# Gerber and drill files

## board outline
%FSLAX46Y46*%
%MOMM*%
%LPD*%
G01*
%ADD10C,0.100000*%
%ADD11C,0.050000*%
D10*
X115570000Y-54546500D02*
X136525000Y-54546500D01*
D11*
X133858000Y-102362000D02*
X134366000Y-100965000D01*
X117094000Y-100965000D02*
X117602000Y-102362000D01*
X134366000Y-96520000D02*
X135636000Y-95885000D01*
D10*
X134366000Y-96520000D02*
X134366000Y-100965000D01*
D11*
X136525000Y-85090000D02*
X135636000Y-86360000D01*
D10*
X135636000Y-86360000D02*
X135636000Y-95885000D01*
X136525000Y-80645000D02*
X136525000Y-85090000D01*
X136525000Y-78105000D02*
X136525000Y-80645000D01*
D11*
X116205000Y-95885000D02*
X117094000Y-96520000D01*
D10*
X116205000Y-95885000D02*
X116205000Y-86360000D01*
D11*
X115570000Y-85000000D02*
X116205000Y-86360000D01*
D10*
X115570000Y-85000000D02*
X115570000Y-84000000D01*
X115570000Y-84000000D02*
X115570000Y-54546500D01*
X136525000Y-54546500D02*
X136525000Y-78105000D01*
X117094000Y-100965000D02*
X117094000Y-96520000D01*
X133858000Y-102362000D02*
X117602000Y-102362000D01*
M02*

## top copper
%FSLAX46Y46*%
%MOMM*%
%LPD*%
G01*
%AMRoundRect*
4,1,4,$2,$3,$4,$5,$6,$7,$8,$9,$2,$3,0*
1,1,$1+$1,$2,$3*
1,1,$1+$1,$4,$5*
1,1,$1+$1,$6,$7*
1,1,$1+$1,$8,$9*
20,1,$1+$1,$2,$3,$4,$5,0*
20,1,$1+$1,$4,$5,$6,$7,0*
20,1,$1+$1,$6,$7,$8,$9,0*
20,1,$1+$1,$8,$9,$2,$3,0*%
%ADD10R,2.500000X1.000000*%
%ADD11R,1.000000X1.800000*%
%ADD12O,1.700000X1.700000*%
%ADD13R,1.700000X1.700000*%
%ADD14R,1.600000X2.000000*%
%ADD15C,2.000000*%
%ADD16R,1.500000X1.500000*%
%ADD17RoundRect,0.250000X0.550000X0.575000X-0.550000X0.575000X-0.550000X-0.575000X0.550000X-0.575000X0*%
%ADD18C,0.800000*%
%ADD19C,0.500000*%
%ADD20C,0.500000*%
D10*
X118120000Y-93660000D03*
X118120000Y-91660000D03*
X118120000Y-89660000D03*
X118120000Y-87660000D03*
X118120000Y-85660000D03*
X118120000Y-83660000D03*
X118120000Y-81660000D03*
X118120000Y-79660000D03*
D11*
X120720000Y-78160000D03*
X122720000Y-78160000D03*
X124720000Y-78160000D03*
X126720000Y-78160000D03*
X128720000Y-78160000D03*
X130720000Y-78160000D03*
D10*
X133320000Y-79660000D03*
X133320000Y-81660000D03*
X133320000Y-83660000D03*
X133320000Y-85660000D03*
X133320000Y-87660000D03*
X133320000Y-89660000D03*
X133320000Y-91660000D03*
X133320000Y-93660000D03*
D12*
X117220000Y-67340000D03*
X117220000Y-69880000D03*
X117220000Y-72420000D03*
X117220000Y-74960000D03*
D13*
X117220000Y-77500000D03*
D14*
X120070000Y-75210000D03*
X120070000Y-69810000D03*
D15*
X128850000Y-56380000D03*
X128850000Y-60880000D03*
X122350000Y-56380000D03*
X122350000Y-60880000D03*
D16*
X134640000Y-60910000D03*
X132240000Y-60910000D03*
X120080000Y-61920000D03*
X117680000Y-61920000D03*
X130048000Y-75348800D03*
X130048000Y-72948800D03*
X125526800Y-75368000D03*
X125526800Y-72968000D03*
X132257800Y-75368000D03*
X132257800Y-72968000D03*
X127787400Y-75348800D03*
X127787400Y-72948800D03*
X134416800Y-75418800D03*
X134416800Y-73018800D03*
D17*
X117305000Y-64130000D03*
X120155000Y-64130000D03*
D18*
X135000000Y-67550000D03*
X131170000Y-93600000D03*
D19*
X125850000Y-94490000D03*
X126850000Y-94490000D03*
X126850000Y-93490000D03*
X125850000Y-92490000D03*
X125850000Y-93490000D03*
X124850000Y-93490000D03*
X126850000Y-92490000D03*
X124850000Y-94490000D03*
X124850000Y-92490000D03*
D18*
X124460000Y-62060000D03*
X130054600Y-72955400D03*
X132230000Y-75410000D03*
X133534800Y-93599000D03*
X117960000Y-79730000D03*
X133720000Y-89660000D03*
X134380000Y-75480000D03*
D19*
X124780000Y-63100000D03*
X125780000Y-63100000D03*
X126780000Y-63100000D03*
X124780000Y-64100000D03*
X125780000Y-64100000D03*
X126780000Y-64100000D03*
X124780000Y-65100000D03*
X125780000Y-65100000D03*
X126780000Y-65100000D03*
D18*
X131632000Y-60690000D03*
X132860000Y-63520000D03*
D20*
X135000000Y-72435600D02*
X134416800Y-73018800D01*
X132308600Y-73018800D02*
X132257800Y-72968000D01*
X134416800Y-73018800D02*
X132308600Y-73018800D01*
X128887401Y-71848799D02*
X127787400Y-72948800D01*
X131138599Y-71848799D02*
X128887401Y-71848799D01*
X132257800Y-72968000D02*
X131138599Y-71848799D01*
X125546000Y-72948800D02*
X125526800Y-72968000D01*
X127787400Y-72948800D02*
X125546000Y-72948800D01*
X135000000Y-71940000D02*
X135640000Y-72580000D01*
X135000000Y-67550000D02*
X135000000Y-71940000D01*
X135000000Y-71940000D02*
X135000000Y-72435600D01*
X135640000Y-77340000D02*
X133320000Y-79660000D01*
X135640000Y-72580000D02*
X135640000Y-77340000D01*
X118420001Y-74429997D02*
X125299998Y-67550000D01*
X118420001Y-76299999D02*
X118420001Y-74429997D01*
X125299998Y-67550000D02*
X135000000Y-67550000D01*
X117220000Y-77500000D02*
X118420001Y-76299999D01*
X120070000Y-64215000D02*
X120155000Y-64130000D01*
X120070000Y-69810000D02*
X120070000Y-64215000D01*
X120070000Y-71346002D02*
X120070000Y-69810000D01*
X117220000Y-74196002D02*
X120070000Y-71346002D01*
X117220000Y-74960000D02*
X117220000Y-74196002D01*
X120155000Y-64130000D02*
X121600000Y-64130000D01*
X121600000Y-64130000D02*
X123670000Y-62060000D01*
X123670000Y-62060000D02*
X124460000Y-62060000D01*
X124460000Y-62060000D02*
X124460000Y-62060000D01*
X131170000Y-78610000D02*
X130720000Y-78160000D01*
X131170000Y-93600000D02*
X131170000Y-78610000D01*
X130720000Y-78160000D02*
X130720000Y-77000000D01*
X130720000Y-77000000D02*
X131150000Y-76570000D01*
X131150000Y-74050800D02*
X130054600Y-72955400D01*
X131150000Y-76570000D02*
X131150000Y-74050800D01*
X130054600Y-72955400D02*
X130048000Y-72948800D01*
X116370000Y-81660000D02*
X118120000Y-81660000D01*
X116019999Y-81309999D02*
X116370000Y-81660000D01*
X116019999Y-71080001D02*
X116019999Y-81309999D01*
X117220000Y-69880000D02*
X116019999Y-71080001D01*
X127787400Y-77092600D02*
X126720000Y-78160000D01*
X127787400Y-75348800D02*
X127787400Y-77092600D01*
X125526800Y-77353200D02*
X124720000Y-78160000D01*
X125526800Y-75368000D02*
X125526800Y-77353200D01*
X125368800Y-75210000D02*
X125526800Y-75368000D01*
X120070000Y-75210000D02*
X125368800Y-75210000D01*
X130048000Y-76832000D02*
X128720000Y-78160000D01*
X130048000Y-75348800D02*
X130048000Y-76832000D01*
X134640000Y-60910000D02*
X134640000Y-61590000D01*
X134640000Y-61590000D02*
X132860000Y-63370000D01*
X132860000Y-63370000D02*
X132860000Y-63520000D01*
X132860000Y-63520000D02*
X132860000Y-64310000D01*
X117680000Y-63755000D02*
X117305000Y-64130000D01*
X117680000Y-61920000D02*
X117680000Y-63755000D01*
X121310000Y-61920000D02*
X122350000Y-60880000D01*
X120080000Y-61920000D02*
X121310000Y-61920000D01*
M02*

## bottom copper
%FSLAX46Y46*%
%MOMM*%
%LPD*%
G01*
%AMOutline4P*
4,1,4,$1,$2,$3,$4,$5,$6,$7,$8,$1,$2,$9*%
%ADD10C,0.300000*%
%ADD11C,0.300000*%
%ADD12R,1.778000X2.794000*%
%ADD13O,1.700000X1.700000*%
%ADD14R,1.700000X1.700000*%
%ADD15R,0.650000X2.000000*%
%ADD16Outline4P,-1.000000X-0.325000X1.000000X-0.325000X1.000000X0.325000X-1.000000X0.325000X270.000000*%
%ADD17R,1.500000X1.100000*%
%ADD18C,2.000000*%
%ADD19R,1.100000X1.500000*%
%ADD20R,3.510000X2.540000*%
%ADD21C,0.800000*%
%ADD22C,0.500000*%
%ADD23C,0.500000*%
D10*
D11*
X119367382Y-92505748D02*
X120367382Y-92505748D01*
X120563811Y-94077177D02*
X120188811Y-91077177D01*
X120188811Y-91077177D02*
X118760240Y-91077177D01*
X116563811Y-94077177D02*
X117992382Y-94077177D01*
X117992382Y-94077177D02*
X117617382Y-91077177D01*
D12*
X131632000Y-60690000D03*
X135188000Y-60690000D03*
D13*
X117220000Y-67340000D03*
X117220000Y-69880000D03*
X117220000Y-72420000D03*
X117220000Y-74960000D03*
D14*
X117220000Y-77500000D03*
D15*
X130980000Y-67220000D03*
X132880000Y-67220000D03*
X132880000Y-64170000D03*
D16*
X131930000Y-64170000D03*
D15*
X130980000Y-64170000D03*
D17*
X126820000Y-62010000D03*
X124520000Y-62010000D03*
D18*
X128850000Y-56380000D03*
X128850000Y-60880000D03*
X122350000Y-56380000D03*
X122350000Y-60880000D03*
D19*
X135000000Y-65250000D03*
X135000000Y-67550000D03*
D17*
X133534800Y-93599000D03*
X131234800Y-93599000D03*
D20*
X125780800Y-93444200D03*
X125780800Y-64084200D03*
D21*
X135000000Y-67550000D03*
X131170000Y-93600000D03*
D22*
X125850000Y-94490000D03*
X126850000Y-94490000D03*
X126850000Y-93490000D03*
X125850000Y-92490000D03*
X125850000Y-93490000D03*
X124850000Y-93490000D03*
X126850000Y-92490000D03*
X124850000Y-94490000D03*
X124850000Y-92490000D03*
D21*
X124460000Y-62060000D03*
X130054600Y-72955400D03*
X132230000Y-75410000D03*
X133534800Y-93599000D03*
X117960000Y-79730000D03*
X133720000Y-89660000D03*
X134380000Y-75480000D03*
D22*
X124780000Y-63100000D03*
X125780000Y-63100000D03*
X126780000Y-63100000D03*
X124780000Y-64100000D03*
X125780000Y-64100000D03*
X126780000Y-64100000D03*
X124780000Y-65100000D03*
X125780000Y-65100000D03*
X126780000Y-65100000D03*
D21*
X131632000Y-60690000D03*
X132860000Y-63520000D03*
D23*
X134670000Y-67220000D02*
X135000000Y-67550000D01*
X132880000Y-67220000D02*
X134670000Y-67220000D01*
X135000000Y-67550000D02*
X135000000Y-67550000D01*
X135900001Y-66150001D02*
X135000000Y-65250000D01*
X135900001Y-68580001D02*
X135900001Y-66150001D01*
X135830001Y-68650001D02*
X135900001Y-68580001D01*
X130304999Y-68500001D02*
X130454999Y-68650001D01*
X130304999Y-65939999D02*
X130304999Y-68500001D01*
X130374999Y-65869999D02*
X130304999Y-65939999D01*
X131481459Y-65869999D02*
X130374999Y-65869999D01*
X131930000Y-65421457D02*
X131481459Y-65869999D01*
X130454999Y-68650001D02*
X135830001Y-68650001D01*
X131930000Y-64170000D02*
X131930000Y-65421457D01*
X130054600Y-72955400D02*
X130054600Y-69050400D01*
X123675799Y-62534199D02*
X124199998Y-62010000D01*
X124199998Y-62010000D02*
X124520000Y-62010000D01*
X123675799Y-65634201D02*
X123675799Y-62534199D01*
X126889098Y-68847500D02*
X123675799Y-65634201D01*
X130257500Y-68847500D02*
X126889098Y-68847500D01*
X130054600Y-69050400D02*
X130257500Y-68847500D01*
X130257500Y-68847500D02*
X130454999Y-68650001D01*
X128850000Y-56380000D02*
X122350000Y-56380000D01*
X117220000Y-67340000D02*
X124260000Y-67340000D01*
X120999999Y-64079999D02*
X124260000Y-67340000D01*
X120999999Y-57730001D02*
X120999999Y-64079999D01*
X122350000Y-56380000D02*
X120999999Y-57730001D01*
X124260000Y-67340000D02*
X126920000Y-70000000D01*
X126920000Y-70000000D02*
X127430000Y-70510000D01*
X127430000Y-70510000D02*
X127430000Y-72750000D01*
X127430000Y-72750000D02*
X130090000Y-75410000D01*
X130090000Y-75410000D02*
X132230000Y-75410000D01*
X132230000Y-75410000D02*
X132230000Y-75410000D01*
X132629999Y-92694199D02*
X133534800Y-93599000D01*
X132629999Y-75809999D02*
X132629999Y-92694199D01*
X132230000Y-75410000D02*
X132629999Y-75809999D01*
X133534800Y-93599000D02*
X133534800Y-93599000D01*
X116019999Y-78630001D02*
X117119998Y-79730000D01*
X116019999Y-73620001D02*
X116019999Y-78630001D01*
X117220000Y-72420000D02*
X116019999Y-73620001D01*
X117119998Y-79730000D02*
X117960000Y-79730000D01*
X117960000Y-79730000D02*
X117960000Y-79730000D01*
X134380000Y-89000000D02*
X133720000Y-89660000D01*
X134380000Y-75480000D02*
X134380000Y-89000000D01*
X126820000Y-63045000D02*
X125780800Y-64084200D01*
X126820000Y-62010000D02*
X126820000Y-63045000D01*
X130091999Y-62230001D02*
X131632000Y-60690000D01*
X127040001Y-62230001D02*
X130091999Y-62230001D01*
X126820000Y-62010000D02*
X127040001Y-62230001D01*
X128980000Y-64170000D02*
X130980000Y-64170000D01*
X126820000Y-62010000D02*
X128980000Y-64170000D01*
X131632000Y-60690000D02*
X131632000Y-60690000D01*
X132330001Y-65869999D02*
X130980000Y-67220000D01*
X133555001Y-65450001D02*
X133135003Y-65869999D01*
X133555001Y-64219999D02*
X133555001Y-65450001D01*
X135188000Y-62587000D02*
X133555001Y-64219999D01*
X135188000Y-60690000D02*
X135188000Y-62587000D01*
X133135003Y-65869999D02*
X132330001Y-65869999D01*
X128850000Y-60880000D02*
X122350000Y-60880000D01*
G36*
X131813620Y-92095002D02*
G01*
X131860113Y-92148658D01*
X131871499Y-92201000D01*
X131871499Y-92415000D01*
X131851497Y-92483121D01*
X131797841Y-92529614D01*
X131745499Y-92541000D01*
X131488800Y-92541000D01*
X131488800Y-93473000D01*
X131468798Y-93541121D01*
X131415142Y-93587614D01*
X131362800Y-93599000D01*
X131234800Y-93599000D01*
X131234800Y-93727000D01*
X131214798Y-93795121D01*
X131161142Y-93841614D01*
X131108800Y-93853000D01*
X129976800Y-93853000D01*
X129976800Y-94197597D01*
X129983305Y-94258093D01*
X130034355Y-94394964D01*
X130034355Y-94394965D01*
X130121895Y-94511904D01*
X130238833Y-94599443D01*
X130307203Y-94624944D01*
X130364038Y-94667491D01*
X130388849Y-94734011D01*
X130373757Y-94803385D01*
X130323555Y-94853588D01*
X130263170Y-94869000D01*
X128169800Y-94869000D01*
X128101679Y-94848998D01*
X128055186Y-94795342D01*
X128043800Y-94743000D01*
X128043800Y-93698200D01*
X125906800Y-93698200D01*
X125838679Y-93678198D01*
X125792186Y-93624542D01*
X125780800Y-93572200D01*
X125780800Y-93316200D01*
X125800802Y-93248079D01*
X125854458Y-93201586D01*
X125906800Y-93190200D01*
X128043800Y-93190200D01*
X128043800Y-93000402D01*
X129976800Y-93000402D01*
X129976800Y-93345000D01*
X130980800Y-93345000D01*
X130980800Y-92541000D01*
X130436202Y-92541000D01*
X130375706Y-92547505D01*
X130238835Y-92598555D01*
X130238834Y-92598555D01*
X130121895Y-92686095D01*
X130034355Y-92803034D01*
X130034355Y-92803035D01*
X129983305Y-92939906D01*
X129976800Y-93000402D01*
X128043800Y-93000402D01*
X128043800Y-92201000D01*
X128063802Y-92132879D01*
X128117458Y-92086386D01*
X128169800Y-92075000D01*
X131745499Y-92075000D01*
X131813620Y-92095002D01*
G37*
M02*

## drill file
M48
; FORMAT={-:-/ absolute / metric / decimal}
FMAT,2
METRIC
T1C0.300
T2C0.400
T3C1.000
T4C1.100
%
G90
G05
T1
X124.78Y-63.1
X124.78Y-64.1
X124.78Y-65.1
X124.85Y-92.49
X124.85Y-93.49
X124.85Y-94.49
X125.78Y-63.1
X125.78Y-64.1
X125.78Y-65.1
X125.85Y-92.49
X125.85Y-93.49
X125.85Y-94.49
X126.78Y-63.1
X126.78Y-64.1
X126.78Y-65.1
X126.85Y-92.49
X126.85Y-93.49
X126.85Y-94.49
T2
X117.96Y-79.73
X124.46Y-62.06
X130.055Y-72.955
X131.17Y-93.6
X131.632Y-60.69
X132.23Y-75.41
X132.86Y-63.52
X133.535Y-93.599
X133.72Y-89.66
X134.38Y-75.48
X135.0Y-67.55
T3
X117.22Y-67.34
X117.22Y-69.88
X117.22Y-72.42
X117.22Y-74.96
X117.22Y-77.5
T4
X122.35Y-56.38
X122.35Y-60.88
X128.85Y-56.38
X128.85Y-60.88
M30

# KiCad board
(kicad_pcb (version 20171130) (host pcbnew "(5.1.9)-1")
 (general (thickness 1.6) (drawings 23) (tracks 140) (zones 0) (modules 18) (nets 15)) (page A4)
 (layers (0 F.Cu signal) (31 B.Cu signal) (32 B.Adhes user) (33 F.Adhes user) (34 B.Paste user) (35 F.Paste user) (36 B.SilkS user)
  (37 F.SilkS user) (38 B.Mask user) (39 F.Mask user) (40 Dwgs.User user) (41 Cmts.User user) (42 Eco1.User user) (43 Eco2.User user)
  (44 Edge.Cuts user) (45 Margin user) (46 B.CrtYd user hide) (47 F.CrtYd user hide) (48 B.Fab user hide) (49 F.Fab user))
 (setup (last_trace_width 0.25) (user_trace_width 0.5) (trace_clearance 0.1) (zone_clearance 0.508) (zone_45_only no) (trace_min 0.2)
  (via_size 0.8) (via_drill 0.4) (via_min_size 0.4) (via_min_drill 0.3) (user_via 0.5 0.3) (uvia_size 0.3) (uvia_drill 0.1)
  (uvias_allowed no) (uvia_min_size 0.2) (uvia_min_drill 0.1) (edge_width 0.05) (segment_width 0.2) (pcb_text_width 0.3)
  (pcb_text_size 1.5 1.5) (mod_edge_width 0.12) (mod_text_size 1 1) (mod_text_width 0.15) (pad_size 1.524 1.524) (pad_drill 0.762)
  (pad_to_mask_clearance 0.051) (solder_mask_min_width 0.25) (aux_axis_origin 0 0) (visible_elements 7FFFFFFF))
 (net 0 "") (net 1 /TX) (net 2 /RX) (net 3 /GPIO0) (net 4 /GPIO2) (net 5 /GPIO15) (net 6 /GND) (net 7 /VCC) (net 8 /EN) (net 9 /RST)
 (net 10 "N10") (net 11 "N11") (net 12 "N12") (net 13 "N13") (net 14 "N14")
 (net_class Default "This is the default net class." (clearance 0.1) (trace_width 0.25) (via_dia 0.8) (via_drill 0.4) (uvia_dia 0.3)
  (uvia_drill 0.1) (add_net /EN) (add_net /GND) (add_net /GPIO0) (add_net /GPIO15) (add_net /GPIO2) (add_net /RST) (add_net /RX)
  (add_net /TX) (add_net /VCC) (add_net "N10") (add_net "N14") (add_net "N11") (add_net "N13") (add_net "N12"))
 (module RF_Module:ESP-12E (layer F.Cu) (at 125.72 90.16 180)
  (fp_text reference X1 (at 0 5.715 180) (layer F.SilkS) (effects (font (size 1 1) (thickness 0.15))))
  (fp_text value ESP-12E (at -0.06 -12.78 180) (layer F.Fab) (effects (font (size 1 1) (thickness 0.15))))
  (pad 22 smd rect (at 7.6 -3.5 180) (size 2.5 1) (layers F.Cu F.Paste F.Mask))
  (pad 21 smd rect (at 7.6 -1.5 180) (size 2.5 1) (layers F.Cu F.Paste F.Mask))
  (pad 20 smd rect (at 7.6 0.5 180) (size 2.5 1) (layers F.Cu F.Paste F.Mask))
  (pad 19 smd rect (at 7.6 2.5 180) (size 2.5 1) (layers F.Cu F.Paste F.Mask))
  (pad 18 smd rect (at 7.6 4.5 180) (size 2.5 1) (layers F.Cu F.Paste F.Mask))
  (pad 17 smd rect (at 7.6 6.5 180) (size 2.5 1) (layers F.Cu F.Paste F.Mask))
  (pad 16 smd rect (at 7.6 8.5 180) (size 2.5 1) (layers F.Cu F.Paste F.Mask) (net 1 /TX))
  (pad 15 smd rect (at 7.6 10.5 180) (size 2.5 1) (layers F.Cu F.Paste F.Mask) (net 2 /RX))
  (pad 14 smd rect (at 5 12 180) (size 1 1.8) (layers F.Cu F.Paste F.Mask))
  (pad 13 smd rect (at 3 12 180) (size 1 1.8) (layers F.Cu F.Paste F.Mask))
  (pad 12 smd rect (at 1 12 180) (size 1 1.8) (layers F.Cu F.Paste F.Mask) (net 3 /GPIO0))
  (pad 11 smd rect (at -1 12 180) (size 1 1.8) (layers F.Cu F.Paste F.Mask) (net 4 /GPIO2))
  (pad 10 smd rect (at -3 12 180) (size 1 1.8) (layers F.Cu F.Paste F.Mask) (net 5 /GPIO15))
  (pad 9 smd rect (at -5 12 180) (size 1 1.8) (layers F.Cu F.Paste F.Mask) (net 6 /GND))
  (pad 8 smd rect (at -7.6 10.5 180) (size 2.5 1) (layers F.Cu F.Paste F.Mask) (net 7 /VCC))
  (pad 7 smd rect (at -7.6 8.5 180) (size 2.5 1) (layers F.Cu F.Paste F.Mask))
  (pad 6 smd rect (at -7.6 6.5 180) (size 2.5 1) (layers F.Cu F.Paste F.Mask))
  (pad 5 smd rect (at -7.6 4.5 180) (size 2.5 1) (layers F.Cu F.Paste F.Mask))
  (pad 4 smd rect (at -7.6 2.5 180) (size 2.5 1) (layers F.Cu F.Paste F.Mask))
  (pad 3 smd rect (at -7.6 0.5 180) (size 2.5 1) (layers F.Cu F.Paste F.Mask) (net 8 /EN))
  (pad 2 smd rect (at -7.6 -1.5 180) (size 2.5 1) (layers F.Cu F.Paste F.Mask))
  (pad 1 smd rect (at -7.6 -3.5 180) (size 2.5 1) (layers F.Cu F.Paste F.Mask) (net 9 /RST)))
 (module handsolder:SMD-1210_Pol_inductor (layer B.Cu) (at 133.41 60.69)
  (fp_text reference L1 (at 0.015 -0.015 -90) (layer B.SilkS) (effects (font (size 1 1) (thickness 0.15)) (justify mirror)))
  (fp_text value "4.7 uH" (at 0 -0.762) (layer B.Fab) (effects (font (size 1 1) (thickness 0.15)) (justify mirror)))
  (pad 1 smd rect (at -1.778 0) (size 1.778 2.794) (layers B.Cu B.Paste B.Mask) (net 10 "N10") (zone_connect 2))
  (pad 2 smd rect (at 1.778 0) (size 1.778 2.794) (layers B.Cu B.Paste B.Mask) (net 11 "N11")))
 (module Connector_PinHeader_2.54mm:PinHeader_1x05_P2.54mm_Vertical (layer F.Cu) (at 117.22 77.5 180)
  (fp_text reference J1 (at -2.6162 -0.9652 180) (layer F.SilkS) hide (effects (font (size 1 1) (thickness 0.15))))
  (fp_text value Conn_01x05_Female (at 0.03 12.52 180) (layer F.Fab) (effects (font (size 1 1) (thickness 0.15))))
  (pad 5 thru_hole oval (at 0 10.16 180) (size 1.7 1.7) (drill 1) (layers *.Cu *.Mask) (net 9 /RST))
  (pad 4 thru_hole oval (at 0 7.62 180) (size 1.7 1.7) (drill 1) (layers *.Cu *.Mask) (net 1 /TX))
  (pad 3 thru_hole oval (at 0 5.08 180) (size 1.7 1.7) (drill 1) (layers *.Cu *.Mask) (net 2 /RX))
  (pad 2 thru_hole oval (at 0 2.54 180) (size 1.7 1.7) (drill 1) (layers *.Cu *.Mask) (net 6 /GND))
  (pad 1 thru_hole rect (at 0 0 180) (size 1.7 1.7) (drill 1) (layers *.Cu *.Mask) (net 7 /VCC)))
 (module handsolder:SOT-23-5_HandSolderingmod (layer B.Cu) (at 131.93 65.72 270)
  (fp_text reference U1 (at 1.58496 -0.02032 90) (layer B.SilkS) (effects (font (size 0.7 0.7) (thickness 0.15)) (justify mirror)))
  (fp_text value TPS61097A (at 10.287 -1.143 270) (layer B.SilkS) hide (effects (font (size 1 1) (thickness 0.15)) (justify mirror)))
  (pad 5 smd rect (at 1.5 0.95 270) (size 2 0.65) (layers B.Cu B.Paste B.Mask) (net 11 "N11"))
  (pad 4 smd rect (at 1.5 -0.95 270) (size 2 0.65) (layers B.Cu B.Paste B.Mask) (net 7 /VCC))
  (pad 3 smd rect (at -1.55 -0.95 270) (size 2 0.65) (layers B.Cu B.Paste B.Mask) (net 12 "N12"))
  (pad 2 smd trapezoid (at -1.55 0 270) (size 2 0.65) (layers B.Cu B.Paste B.Mask) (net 6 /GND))
  (pad 1 smd rect (at -1.55 0.95 270) (size 2 0.65) (layers B.Cu B.Paste B.Mask) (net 10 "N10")))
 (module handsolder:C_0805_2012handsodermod (layer B.Cu) (at 125.67 62.01)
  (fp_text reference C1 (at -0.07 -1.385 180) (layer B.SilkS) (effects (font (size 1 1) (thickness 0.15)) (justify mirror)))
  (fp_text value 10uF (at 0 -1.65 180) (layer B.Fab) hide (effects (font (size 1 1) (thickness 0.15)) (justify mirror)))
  (pad 2 smd rect (at 1.15 0) (size 1.5 1.1) (layers B.Cu B.Paste B.Mask) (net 10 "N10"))
  (pad 1 smd rect (at -1.15 0) (size 1.5 1.1) (layers B.Cu B.Paste B.Mask) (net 6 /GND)))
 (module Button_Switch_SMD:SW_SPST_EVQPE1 (layer F.Cu) (at 120.07 72.51 90)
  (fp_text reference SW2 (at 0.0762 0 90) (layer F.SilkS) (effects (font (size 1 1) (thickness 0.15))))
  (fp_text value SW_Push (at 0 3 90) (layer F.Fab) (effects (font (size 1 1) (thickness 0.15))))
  (pad 1 smd rect (at -2.7 0 90) (size 2 1.6) (layers F.Cu F.Paste F.Mask) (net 3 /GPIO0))
  (pad 2 smd rect (at 2.7 0 90) (size 2 1.6) (layers F.Cu F.Paste F.Mask) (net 6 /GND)))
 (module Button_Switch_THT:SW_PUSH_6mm (layer F.Cu) (at 122.35 56.38)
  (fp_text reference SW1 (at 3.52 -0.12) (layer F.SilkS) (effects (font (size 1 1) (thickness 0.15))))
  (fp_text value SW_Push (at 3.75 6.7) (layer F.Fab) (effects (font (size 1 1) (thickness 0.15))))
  (pad 1 thru_hole circle (at 6.5 0 90) (size 2 2) (drill 1.1) (layers *.Cu *.Mask) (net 9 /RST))
  (pad 2 thru_hole circle (at 6.5 4.5 90) (size 2 2) (drill 1.1) (layers *.Cu *.Mask) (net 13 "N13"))
  (pad 1 thru_hole circle (at 0 0 90) (size 2 2) (drill 1.1) (layers *.Cu *.Mask) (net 9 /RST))
  (pad 2 thru_hole circle (at 0 4.5 90) (size 2 2) (drill 1.1) (layers *.Cu *.Mask) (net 13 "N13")))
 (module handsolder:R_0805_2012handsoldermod (layer F.Cu) (at 133.44 60.91)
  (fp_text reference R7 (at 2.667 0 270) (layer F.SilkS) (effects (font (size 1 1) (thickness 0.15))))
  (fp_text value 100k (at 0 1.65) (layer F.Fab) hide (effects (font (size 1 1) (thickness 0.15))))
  (pad 2 smd rect (at 1.2 0) (size 1.5 1.5) (layers F.Cu F.Paste F.Mask) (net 12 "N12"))
  (pad 1 smd rect (at -1.2 0) (size 1.5 1.5) (layers F.Cu F.Paste F.Mask) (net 10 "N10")))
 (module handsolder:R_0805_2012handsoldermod (layer F.Cu) (at 118.88 61.92)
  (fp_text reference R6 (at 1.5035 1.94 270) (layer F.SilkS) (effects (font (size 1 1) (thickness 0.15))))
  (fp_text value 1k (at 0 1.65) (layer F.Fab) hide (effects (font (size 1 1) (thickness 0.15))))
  (pad 2 smd rect (at 1.2 0) (size 1.5 1.5) (layers F.Cu F.Paste F.Mask) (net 13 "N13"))
  (pad 1 smd rect (at -1.2 0) (size 1.5 1.5) (layers F.Cu F.Paste F.Mask) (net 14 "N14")))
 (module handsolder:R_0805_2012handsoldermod (layer F.Cu) (at 130.048 74.1488 270)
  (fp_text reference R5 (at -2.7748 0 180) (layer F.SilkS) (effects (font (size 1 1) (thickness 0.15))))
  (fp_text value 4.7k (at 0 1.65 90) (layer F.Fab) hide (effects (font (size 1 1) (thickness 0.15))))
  (pad 2 smd rect (at 1.2 0 270) (size 1.5 1.5) (layers F.Cu F.Paste F.Mask) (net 5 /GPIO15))
  (pad 1 smd rect (at -1.2 0 270) (size 1.5 1.5) (layers F.Cu F.Paste F.Mask) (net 6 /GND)))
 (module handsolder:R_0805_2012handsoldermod (layer F.Cu) (at 125.5268 74.168 270)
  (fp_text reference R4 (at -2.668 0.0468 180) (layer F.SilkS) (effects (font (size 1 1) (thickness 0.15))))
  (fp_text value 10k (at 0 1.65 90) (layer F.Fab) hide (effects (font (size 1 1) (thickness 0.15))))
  (pad 2 smd rect (at 1.2 0 270) (size 1.5 1.5) (layers F.Cu F.Paste F.Mask) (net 3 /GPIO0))
  (pad 1 smd rect (at -1.2 0 270) (size 1.5 1.5) (layers F.Cu F.Paste F.Mask) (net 7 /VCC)))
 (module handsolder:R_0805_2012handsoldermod (layer F.Cu) (at 132.2578 74.168 270)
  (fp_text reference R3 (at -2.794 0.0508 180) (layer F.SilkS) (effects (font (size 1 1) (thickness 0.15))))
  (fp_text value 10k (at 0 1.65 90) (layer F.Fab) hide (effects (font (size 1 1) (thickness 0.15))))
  (pad 2 smd rect (at 1.2 0 270) (size 1.5 1.5) (layers F.Cu F.Paste F.Mask) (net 9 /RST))
  (pad 1 smd rect (at -1.2 0 270) (size 1.5 1.5) (layers F.Cu F.Paste F.Mask) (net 7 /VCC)))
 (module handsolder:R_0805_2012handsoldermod (layer F.Cu) (at 127.7874 74.1488 270)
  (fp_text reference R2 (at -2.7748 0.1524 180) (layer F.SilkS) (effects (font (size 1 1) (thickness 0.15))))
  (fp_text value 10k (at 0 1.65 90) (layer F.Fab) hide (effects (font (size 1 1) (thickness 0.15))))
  (pad 2 smd rect (at 1.2 0 270) (size 1.5 1.5) (layers F.Cu F.Paste F.Mask) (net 4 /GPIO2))
  (pad 1 smd rect (at -1.2 0 270) (size 1.5 1.5) (layers F.Cu F.Paste F.Mask) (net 7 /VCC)))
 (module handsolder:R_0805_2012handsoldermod (layer F.Cu) (at 134.4168 74.2188 270)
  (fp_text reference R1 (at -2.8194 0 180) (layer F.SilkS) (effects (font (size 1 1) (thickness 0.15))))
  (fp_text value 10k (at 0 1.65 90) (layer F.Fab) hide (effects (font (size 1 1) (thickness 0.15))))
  (pad 2 smd rect (at 1.2 0 270) (size 1.5 1.5) (layers F.Cu F.Paste F.Mask) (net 8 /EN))
  (pad 1 smd rect (at -1.2 0 270) (size 1.5 1.5) (layers F.Cu F.Paste F.Mask) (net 7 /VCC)))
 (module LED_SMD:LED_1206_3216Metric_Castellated (layer F.Cu) (at 118.73 64.13 180)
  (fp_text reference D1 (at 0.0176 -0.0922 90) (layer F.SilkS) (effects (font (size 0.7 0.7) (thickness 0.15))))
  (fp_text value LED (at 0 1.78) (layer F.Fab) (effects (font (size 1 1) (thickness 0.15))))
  (pad 2 smd roundrect (at 1.425 0 180) (size 1.6 1.65) (layers F.Cu F.Paste F.Mask) (roundrect_rratio 0.15625) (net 14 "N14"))
  (pad 1 smd roundrect (at -1.425 0 180) (size 1.6 1.65) (layers F.Cu F.Paste F.Mask) (roundrect_rratio 0.15625) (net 6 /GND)))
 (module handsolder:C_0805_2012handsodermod (layer B.Cu) (at 135 66.4 90)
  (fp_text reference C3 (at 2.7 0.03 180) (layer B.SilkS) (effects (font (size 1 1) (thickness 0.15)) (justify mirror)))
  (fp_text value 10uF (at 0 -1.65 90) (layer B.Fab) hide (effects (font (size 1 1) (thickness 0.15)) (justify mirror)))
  (pad 2 smd rect (at 1.15 0 90) (size 1.5 1.1) (layers B.Cu B.Paste B.Mask) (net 6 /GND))
  (pad 1 smd rect (at -1.15 0 90) (size 1.5 1.1) (layers B.Cu B.Paste B.Mask) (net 7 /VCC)))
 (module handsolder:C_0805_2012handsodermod (layer B.Cu) (at 132.3848 93.599)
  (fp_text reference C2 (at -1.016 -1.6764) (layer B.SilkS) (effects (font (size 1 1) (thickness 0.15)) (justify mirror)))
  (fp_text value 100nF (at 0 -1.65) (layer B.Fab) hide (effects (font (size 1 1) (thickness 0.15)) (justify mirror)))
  (pad 2 smd rect (at 1.15 0) (size 1.5 1.1) (layers B.Cu B.Paste B.Mask) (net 9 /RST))
  (pad 1 smd rect (at -1.15 0) (size 1.5 1.1) (layers B.Cu B.Paste B.Mask) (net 6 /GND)))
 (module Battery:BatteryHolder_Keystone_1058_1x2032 (layer B.Cu) (at 125.7808 78.7642 270)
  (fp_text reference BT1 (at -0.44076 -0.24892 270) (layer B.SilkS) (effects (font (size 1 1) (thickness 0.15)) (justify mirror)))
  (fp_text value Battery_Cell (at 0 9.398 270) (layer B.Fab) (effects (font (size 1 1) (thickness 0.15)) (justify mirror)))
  (pad 2 smd rect (at 14.68 0 270) (size 2.54 3.51) (layers B.Cu B.Paste B.Mask) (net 6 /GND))
  (pad 1 smd rect (at -14.68 0 270) (size 2.54 3.51) (layers B.Cu B.Paste B.Mask) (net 10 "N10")))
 (gr_line (start 115.57 54.5465) (end 136.525 54.5465) (layer Edge.Cuts) (width 0.1))
 (gr_line (start 133.858 102.362) (end 134.366 100.965) (layer Edge.Cuts) (width 0.05))
 (gr_line (start 117.094 100.965) (end 117.602 102.362) (layer Edge.Cuts) (width 0.05))
 (gr_line (start 134.366 96.52) (end 135.636 95.885) (layer Edge.Cuts) (width 0.05))
 (gr_line (start 134.366 96.52) (end 134.366 100.965) (layer Edge.Cuts) (width 0.1))
 (gr_line (start 136.525 85.09) (end 135.636 86.36) (layer Edge.Cuts) (width 0.05))
 (gr_line (start 135.636 86.36) (end 135.636 95.885) (layer Edge.Cuts) (width 0.1))
 (gr_line (start 136.525 80.645) (end 136.525 85.09) (layer Edge.Cuts) (width 0.1))
 (gr_line (start 136.525 78.105) (end 136.525 80.645) (layer Edge.Cuts) (width 0.1))
 (gr_line (start 116.205 95.885) (end 117.094 96.52) (layer Edge.Cuts) (width 0.05))
 (gr_line (start 116.205 95.885) (end 116.205 86.36) (layer Edge.Cuts) (width 0.1))
 (gr_line (start 115.57 85) (end 116.205 86.36) (layer Edge.Cuts) (width 0.05))
 (gr_line (start 115.57 85) (end 115.57 84) (layer Edge.Cuts) (width 0.1))
 (gr_line (start 115.57 84) (end 115.57 54.5465) (layer Edge.Cuts) (width 0.1))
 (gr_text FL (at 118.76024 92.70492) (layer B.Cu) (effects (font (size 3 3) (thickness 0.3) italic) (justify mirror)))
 (gr_line (start 136.525 54.5465) (end 136.525 78.105) (layer Edge.Cuts) (width 0.1))
 (gr_line (start 117.094 100.965) (end 117.094 96.52) (layer Edge.Cuts) (width 0.1))
 (gr_line (start 133.858 102.362) (end 117.602 102.362) (layer Edge.Cuts) (width 0.1))
 (segment (start 134.67 67.22) (end 135 67.55) (width 0.5) (layer B.Cu) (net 7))
 (segment (start 132.88 67.22) (end 134.67 67.22) (width 0.5) (layer B.Cu) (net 7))
 (segment (start 135 67.55) (end 135 67.55) (width 0.5) (layer B.Cu) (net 7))
 (via (at 135 67.55) (size 0.8) (drill 0.4) (layers F.Cu B.Cu) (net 7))
 (segment (start 135 72.4356) (end 134.4168 73.0188) (width 0.5) (layer F.Cu) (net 7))
 (segment (start 132.3086 73.0188) (end 132.2578 72.968) (width 0.5) (layer F.Cu) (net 7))
 (segment (start 134.4168 73.0188) (end 132.3086 73.0188) (width 0.5) (layer F.Cu) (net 7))
 (segment (start 128.887401 71.848799) (end 127.7874 72.9488) (width 0.5) (layer F.Cu) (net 7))
 (segment (start 131.138599 71.848799) (end 128.887401 71.848799) (width 0.5) (layer F.Cu) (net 7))
 (segment (start 132.2578 72.968) (end 131.138599 71.848799) (width 0.5) (layer F.Cu) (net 7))
 (segment (start 125.546 72.9488) (end 125.5268 72.968) (width 0.5) (layer F.Cu) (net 7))
 (segment (start 127.7874 72.9488) (end 125.546 72.9488) (width 0.5) (layer F.Cu) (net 7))
 (segment (start 135 71.94) (end 135.64 72.58) (width 0.5) (layer F.Cu) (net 7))
 (segment (start 135 67.55) (end 135 71.94) (width 0.5) (layer F.Cu) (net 7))
 (segment (start 135 71.94) (end 135 72.4356) (width 0.5) (layer F.Cu) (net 7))
 (segment (start 135.64 77.34) (end 133.32 79.66) (width 0.5) (layer F.Cu) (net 7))
 (segment (start 135.64 72.58) (end 135.64 77.34) (width 0.5) (layer F.Cu) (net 7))
 (segment (start 118.420001 74.429997) (end 125.299998 67.55) (width 0.5) (layer F.Cu) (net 7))
 (segment (start 118.420001 76.299999) (end 118.420001 74.429997) (width 0.5) (layer F.Cu) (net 7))
 (segment (start 125.299998 67.55) (end 135 67.55) (width 0.5) (layer F.Cu) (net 7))
 (segment (start 117.22 77.5) (end 118.420001 76.299999) (width 0.5) (layer F.Cu) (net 7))
 (via (at 131.17 93.6) (size 0.8) (drill 0.4) (layers F.Cu B.Cu) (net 6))
 (via (at 125.85 94.49) (size 0.5) (drill 0.3) (layers F.Cu B.Cu) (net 6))
 (via (at 126.85 94.49) (size 0.5) (drill 0.3) (layers F.Cu B.Cu) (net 6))
 (via (at 126.85 93.49) (size 0.5) (drill 0.3) (layers F.Cu B.Cu) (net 6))
 (via (at 125.85 92.49) (size 0.5) (drill 0.3) (layers F.Cu B.Cu) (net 6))
 (via (at 125.85 93.49) (size 0.5) (drill 0.3) (layers F.Cu B.Cu) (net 6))
 (via (at 124.85 93.49) (size 0.5) (drill 0.3) (layers F.Cu B.Cu) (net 6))
 (via (at 126.85 92.49) (size 0.5) (drill 0.3) (layers F.Cu B.Cu) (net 6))
 (via (at 124.85 94.49) (size 0.5) (drill 0.3) (layers F.Cu B.Cu) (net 6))
 (via (at 124.85 92.49) (size 0.5) (drill 0.3) (layers F.Cu B.Cu) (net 6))
 (segment (start 120.07 64.215) (end 120.155 64.13) (width 0.5) (layer F.Cu) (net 6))
 (segment (start 120.07 69.81) (end 120.07 64.215) (width 0.5) (layer F.Cu) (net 6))
 (segment (start 135.900001 66.150001) (end 135 65.25) (width 0.5) (layer B.Cu) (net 6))
 (segment (start 135.900001 68.580001) (end 135.900001 66.150001) (width 0.5) (layer B.Cu) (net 6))
 (segment (start 135.830001 68.650001) (end 135.900001 68.580001) (width 0.5) (layer B.Cu) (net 6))
 (segment (start 130.304999 68.500001) (end 130.454999 68.650001) (width 0.5) (layer B.Cu) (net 6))
 (segment (start 130.304999 65.939999) (end 130.304999 68.500001) (width 0.5) (layer B.Cu) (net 6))
 (segment (start 130.374999 65.869999) (end 130.304999 65.939999) (width 0.5) (layer B.Cu) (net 6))
 (segment (start 131.481459 65.869999) (end 130.374999 65.869999) (width 0.5) (layer B.Cu) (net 6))
 (segment (start 131.93 65.421457) (end 131.481459 65.869999) (width 0.5) (layer B.Cu) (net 6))
 (segment (start 130.454999 68.650001) (end 135.830001 68.650001) (width 0.5) (layer B.Cu) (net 6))
 (segment (start 131.93 64.17) (end 131.93 65.421457) (width 0.5) (layer B.Cu) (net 6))
 (segment (start 120.07 71.346002) (end 120.07 69.81) (width 0.5) (layer F.Cu) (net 6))
 (segment (start 117.22 74.196002) (end 120.07 71.346002) (width 0.5) (layer F.Cu) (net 6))
 (segment (start 117.22 74.96) (end 117.22 74.196002) (width 0.5) (layer F.Cu) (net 6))
 (segment (start 120.155 64.13) (end 121.6 64.13) (width 0.5) (layer F.Cu) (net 6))
 (segment (start 121.6 64.13) (end 123.67 62.06) (width 0.5) (layer F.Cu) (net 6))
 (segment (start 123.67 62.06) (end 124.46 62.06) (width 0.5) (layer F.Cu) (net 6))
 (segment (start 124.46 62.06) (end 124.46 62.06) (width 0.5) (layer F.Cu) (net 6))
 (via (at 124.46 62.06) (size 0.8) (drill 0.4) (layers F.Cu B.Cu) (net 6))
 (segment (start 131.17 78.61) (end 130.72 78.16) (width 0.5) (layer F.Cu) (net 6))
 (segment (start 131.17 93.6) (end 131.17 78.61) (width 0.5) (layer F.Cu) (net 6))
 (segment (start 130.72 78.16) (end 130.72 77) (width 0.5) (layer F.Cu) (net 6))
 (segment (start 130.72 77) (end 131.15 76.57) (width 0.5) (layer F.Cu) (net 6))
 (segment (start 131.15 74.0508) (end 130.0546 72.9554) (width 0.5) (layer F.Cu) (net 6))
 (segment (start 131.15 76.57) (end 131.15 74.0508) (width 0.5) (layer F.Cu) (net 6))
 (segment (start 130.0546 72.9554) (end 130.048 72.9488) (width 0.5) (layer F.Cu) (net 6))
 (via (at 130.0546 72.9554) (size 0.8) (drill 0.4) (layers F.Cu B.Cu) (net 6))
 (segment (start 130.0546 72.9554) (end 130.0546 69.0504) (width 0.5) (layer B.Cu) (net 6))
 (segment (start 123.675799 62.534199) (end 124.199998 62.01) (width 0.5) (layer B.Cu) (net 6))
 (segment (start 124.199998 62.01) (end 124.52 62.01) (width 0.5) (layer B.Cu) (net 6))
 (segment (start 123.675799 65.634201) (end 123.675799 62.534199) (width 0.5) (layer B.Cu) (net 6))
 (segment (start 126.889098 68.8475) (end 123.675799 65.634201) (width 0.5) (layer B.Cu) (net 6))
 (segment (start 130.2575 68.8475) (end 126.889098 68.8475) (width 0.5) (layer B.Cu) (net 6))
 (segment (start 130.0546 69.0504) (end 130.2575 68.8475) (width 0.5) (layer B.Cu) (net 6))
 (segment (start 130.2575 68.8475) (end 130.454999 68.650001) (width 0.5) (layer B.Cu) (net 6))
 (segment (start 128.85 56.38) (end 122.35 56.38) (width 0.5) (layer B.Cu) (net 9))
 (segment (start 117.22 67.34) (end 124.26 67.34) (width 0.5) (layer B.Cu) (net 9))
 (segment (start 120.999999 64.079999) (end 124.26 67.34) (width 0.5) (layer B.Cu) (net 9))
 (segment (start 120.999999 57.730001) (end 120.999999 64.079999) (width 0.5) (layer B.Cu) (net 9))
 (segment (start 122.35 56.38) (end 120.999999 57.730001) (width 0.5) (layer B.Cu) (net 9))
 (segment (start 124.26 67.34) (end 126.92 70) (width 0.5) (layer B.Cu) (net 9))
 (segment (start 126.92 70) (end 127.43 70.51) (width 0.5) (layer B.Cu) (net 9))
 (segment (start 127.43 70.51) (end 127.43 72.75) (width 0.5) (layer B.Cu) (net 9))
 (segment (start 127.43 72.75) (end 130.09 75.41) (width 0.5) (layer B.Cu) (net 9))
 (segment (start 130.09 75.41) (end 132.23 75.41) (width 0.5) (layer B.Cu) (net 9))
 (segment (start 132.23 75.41) (end 132.23 75.41) (width 0.5) (layer B.Cu) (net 9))
 (via (at 132.23 75.41) (size 0.8) (drill 0.4) (layers F.Cu B.Cu) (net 9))
 (segment (start 132.629999 92.694199) (end 133.5348 93.599) (width 0.5) (layer B.Cu) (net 9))
 (segment (start 132.629999 75.809999) (end 132.629999 92.694199) (width 0.5) (layer B.Cu) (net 9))
 (segment (start 132.23 75.41) (end 132.629999 75.809999) (width 0.5) (layer B.Cu) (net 9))
 (segment (start 133.5348 93.599) (end 133.5348 93.599) (width 0.5) (layer B.Cu) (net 9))
 (via (at 133.5348 93.599) (size 0.8) (drill 0.4) (layers F.Cu B.Cu) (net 9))
 (segment (start 116.019999 78.630001) (end 117.119998 79.73) (width 0.5) (layer B.Cu) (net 2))
 (segment (start 116.019999 73.620001) (end 116.019999 78.630001) (width 0.5) (layer B.Cu) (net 2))
 (segment (start 117.22 72.42) (end 116.019999 73.620001) (width 0.5) (layer B.Cu) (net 2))
 (segment (start 117.119998 79.73) (end 117.96 79.73) (width 0.5) (layer B.Cu) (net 2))
 (segment (start 117.96 79.73) (end 117.96 79.73) (width 0.5) (layer B.Cu) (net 2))
 (via (at 117.96 79.73) (size 0.8) (drill 0.4) (layers F.Cu B.Cu) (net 2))
 (segment (start 116.37 81.66) (end 118.12 81.66) (width 0.5) (layer F.Cu) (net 1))
 (segment (start 116.019999 81.309999) (end 116.37 81.66) (width 0.5) (layer F.Cu) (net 1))
 (segment (start 116.019999 71.080001) (end 116.019999 81.309999) (width 0.5) (layer F.Cu) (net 1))
 (segment (start 117.22 69.88) (end 116.019999 71.080001) (width 0.5) (layer F.Cu) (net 1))
 (via (at 133.72 89.66) (size 0.8) (drill 0.4) (layers F.Cu B.Cu) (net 8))
 (via (at 134.38 75.48) (size 0.8) (drill 0.4) (layers F.Cu B.Cu) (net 8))
 (segment (start 134.38 89) (end 133.72 89.66) (width 0.5) (layer B.Cu) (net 8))
 (segment (start 134.38 75.48) (end 134.38 89) (width 0.5) (layer B.Cu) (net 8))
 (segment (start 127.7874 77.0926) (end 126.72 78.16) (width 0.5) (layer F.Cu) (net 4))
 (segment (start 127.7874 75.3488) (end 127.7874 77.0926) (width 0.5) (layer F.Cu) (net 4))
 (segment (start 125.5268 77.3532) (end 124.72 78.16) (width 0.5) (layer F.Cu) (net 3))
 (segment (start 125.5268 75.368) (end 125.5268 77.3532) (width 0.5) (layer F.Cu) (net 3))
 (segment (start 125.3688 75.21) (end 125.5268 75.368) (width 0.5) (layer F.Cu) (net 3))
 (segment (start 120.07 75.21) (end 125.3688 75.21) (width 0.5) (layer F.Cu) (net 3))
 (via (at 124.78 63.1) (size 0.5) (drill 0.3) (layers F.Cu B.Cu) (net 10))
 (via (at 125.78 63.1) (size 0.5) (drill 0.3) (layers F.Cu B.Cu) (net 10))
 (via (at 126.78 63.1) (size 0.5) (drill 0.3) (layers F.Cu B.Cu) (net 10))
 (via (at 124.78 64.1) (size 0.5) (drill 0.3) (layers F.Cu B.Cu) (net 10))
 (via (at 125.78 64.1) (size 0.5) (drill 0.3) (layers F.Cu B.Cu) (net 10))
 (via (at 126.78 64.1) (size 0.5) (drill 0.3) (layers F.Cu B.Cu) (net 10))
 (via (at 124.78 65.1) (size 0.5) (drill 0.3) (layers F.Cu B.Cu) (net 10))
 (via (at 125.78 65.1) (size 0.5) (drill 0.3) (layers F.Cu B.Cu) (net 10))
 (via (at 126.78 65.1) (size 0.5) (drill 0.3) (layers F.Cu B.Cu) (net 10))
 (segment (start 126.82 63.045) (end 125.7808 64.0842) (width 0.5) (layer B.Cu) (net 10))
 (segment (start 126.82 62.01) (end 126.82 63.045) (width 0.5) (layer B.Cu) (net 10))
 (segment (start 130.091999 62.230001) (end 131.632 60.69) (width 0.5) (layer B.Cu) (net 10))
 (segment (start 127.040001 62.230001) (end 130.091999 62.230001) (width 0.5) (layer B.Cu) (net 10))
 (segment (start 126.82 62.01) (end 127.040001 62.230001) (width 0.5) (layer B.Cu) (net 10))
 (segment (start 128.98 64.17) (end 130.98 64.17) (width 0.5) (layer B.Cu) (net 10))
 (segment (start 126.82 62.01) (end 128.98 64.17) (width 0.5) (layer B.Cu) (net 10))
 (segment (start 131.632 60.69) (end 131.632 60.69) (width 0.5) (layer B.Cu) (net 10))
 (via (at 131.632 60.69) (size 0.8) (drill 0.4) (layers F.Cu B.Cu) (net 10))
 (segment (start 132.330001 65.869999) (end 130.98 67.22) (width 0.5) (layer B.Cu) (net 11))
 (segment (start 133.555001 65.450001) (end 133.135003 65.869999) (width 0.5) (layer B.Cu) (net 11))
 (segment (start 133.555001 64.219999) (end 133.555001 65.450001) (width 0.5) (layer B.Cu) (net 11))
 (segment (start 135.188 62.587) (end 133.555001 64.219999) (width 0.5) (layer B.Cu) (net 11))
 (segment (start 135.188 60.69) (end 135.188 62.587) (width 0.5) (layer B.Cu) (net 11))
 (segment (start 133.135003 65.869999) (end 132.330001 65.869999) (width 0.5) (layer B.Cu) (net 11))
 (segment (start 130.048 76.832) (end 128.72 78.16) (width 0.5) (layer F.Cu) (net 5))
 (segment (start 130.048 75.3488) (end 130.048 76.832) (width 0.5) (layer F.Cu) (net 5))
 (segment (start 134.64 60.91) (end 134.64 61.59) (width 0.5) (layer F.Cu) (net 12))
 (segment (start 134.64 61.59) (end 132.86 63.37) (width 0.5) (layer F.Cu) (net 12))
 (segment (start 132.86 63.37) (end 132.86 63.52) (width 0.5) (layer F.Cu) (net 12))
 (segment (start 132.86 63.52) (end 132.86 64.31) (width 0.5) (layer F.Cu) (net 12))
 (via (at 132.86 63.52) (size 0.8) (drill 0.4) (layers F.Cu B.Cu) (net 12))
 (segment (start 117.68 63.755) (end 117.305 64.13) (width 0.5) (layer F.Cu) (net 14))
 (segment (start 117.68 61.92) (end 117.68 63.755) (width 0.5) (layer F.Cu) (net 14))
 (segment (start 128.85 60.88) (end 122.35 60.88) (width 0.5) (layer B.Cu) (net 13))
 (segment (start 121.31 61.92) (end 122.35 60.88) (width 0.5) (layer F.Cu) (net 13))
 (segment (start 120.08 61.92) (end 121.31 61.92) (width 0.5) (layer F.Cu) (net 13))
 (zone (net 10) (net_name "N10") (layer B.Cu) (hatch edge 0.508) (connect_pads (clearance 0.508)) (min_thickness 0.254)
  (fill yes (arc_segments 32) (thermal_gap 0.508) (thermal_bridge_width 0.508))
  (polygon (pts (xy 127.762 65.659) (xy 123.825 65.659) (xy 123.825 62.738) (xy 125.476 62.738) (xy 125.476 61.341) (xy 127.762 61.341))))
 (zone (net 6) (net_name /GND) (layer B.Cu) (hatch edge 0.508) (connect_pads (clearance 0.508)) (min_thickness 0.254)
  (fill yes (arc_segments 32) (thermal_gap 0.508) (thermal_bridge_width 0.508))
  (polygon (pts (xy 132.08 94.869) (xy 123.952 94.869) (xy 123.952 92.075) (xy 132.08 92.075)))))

